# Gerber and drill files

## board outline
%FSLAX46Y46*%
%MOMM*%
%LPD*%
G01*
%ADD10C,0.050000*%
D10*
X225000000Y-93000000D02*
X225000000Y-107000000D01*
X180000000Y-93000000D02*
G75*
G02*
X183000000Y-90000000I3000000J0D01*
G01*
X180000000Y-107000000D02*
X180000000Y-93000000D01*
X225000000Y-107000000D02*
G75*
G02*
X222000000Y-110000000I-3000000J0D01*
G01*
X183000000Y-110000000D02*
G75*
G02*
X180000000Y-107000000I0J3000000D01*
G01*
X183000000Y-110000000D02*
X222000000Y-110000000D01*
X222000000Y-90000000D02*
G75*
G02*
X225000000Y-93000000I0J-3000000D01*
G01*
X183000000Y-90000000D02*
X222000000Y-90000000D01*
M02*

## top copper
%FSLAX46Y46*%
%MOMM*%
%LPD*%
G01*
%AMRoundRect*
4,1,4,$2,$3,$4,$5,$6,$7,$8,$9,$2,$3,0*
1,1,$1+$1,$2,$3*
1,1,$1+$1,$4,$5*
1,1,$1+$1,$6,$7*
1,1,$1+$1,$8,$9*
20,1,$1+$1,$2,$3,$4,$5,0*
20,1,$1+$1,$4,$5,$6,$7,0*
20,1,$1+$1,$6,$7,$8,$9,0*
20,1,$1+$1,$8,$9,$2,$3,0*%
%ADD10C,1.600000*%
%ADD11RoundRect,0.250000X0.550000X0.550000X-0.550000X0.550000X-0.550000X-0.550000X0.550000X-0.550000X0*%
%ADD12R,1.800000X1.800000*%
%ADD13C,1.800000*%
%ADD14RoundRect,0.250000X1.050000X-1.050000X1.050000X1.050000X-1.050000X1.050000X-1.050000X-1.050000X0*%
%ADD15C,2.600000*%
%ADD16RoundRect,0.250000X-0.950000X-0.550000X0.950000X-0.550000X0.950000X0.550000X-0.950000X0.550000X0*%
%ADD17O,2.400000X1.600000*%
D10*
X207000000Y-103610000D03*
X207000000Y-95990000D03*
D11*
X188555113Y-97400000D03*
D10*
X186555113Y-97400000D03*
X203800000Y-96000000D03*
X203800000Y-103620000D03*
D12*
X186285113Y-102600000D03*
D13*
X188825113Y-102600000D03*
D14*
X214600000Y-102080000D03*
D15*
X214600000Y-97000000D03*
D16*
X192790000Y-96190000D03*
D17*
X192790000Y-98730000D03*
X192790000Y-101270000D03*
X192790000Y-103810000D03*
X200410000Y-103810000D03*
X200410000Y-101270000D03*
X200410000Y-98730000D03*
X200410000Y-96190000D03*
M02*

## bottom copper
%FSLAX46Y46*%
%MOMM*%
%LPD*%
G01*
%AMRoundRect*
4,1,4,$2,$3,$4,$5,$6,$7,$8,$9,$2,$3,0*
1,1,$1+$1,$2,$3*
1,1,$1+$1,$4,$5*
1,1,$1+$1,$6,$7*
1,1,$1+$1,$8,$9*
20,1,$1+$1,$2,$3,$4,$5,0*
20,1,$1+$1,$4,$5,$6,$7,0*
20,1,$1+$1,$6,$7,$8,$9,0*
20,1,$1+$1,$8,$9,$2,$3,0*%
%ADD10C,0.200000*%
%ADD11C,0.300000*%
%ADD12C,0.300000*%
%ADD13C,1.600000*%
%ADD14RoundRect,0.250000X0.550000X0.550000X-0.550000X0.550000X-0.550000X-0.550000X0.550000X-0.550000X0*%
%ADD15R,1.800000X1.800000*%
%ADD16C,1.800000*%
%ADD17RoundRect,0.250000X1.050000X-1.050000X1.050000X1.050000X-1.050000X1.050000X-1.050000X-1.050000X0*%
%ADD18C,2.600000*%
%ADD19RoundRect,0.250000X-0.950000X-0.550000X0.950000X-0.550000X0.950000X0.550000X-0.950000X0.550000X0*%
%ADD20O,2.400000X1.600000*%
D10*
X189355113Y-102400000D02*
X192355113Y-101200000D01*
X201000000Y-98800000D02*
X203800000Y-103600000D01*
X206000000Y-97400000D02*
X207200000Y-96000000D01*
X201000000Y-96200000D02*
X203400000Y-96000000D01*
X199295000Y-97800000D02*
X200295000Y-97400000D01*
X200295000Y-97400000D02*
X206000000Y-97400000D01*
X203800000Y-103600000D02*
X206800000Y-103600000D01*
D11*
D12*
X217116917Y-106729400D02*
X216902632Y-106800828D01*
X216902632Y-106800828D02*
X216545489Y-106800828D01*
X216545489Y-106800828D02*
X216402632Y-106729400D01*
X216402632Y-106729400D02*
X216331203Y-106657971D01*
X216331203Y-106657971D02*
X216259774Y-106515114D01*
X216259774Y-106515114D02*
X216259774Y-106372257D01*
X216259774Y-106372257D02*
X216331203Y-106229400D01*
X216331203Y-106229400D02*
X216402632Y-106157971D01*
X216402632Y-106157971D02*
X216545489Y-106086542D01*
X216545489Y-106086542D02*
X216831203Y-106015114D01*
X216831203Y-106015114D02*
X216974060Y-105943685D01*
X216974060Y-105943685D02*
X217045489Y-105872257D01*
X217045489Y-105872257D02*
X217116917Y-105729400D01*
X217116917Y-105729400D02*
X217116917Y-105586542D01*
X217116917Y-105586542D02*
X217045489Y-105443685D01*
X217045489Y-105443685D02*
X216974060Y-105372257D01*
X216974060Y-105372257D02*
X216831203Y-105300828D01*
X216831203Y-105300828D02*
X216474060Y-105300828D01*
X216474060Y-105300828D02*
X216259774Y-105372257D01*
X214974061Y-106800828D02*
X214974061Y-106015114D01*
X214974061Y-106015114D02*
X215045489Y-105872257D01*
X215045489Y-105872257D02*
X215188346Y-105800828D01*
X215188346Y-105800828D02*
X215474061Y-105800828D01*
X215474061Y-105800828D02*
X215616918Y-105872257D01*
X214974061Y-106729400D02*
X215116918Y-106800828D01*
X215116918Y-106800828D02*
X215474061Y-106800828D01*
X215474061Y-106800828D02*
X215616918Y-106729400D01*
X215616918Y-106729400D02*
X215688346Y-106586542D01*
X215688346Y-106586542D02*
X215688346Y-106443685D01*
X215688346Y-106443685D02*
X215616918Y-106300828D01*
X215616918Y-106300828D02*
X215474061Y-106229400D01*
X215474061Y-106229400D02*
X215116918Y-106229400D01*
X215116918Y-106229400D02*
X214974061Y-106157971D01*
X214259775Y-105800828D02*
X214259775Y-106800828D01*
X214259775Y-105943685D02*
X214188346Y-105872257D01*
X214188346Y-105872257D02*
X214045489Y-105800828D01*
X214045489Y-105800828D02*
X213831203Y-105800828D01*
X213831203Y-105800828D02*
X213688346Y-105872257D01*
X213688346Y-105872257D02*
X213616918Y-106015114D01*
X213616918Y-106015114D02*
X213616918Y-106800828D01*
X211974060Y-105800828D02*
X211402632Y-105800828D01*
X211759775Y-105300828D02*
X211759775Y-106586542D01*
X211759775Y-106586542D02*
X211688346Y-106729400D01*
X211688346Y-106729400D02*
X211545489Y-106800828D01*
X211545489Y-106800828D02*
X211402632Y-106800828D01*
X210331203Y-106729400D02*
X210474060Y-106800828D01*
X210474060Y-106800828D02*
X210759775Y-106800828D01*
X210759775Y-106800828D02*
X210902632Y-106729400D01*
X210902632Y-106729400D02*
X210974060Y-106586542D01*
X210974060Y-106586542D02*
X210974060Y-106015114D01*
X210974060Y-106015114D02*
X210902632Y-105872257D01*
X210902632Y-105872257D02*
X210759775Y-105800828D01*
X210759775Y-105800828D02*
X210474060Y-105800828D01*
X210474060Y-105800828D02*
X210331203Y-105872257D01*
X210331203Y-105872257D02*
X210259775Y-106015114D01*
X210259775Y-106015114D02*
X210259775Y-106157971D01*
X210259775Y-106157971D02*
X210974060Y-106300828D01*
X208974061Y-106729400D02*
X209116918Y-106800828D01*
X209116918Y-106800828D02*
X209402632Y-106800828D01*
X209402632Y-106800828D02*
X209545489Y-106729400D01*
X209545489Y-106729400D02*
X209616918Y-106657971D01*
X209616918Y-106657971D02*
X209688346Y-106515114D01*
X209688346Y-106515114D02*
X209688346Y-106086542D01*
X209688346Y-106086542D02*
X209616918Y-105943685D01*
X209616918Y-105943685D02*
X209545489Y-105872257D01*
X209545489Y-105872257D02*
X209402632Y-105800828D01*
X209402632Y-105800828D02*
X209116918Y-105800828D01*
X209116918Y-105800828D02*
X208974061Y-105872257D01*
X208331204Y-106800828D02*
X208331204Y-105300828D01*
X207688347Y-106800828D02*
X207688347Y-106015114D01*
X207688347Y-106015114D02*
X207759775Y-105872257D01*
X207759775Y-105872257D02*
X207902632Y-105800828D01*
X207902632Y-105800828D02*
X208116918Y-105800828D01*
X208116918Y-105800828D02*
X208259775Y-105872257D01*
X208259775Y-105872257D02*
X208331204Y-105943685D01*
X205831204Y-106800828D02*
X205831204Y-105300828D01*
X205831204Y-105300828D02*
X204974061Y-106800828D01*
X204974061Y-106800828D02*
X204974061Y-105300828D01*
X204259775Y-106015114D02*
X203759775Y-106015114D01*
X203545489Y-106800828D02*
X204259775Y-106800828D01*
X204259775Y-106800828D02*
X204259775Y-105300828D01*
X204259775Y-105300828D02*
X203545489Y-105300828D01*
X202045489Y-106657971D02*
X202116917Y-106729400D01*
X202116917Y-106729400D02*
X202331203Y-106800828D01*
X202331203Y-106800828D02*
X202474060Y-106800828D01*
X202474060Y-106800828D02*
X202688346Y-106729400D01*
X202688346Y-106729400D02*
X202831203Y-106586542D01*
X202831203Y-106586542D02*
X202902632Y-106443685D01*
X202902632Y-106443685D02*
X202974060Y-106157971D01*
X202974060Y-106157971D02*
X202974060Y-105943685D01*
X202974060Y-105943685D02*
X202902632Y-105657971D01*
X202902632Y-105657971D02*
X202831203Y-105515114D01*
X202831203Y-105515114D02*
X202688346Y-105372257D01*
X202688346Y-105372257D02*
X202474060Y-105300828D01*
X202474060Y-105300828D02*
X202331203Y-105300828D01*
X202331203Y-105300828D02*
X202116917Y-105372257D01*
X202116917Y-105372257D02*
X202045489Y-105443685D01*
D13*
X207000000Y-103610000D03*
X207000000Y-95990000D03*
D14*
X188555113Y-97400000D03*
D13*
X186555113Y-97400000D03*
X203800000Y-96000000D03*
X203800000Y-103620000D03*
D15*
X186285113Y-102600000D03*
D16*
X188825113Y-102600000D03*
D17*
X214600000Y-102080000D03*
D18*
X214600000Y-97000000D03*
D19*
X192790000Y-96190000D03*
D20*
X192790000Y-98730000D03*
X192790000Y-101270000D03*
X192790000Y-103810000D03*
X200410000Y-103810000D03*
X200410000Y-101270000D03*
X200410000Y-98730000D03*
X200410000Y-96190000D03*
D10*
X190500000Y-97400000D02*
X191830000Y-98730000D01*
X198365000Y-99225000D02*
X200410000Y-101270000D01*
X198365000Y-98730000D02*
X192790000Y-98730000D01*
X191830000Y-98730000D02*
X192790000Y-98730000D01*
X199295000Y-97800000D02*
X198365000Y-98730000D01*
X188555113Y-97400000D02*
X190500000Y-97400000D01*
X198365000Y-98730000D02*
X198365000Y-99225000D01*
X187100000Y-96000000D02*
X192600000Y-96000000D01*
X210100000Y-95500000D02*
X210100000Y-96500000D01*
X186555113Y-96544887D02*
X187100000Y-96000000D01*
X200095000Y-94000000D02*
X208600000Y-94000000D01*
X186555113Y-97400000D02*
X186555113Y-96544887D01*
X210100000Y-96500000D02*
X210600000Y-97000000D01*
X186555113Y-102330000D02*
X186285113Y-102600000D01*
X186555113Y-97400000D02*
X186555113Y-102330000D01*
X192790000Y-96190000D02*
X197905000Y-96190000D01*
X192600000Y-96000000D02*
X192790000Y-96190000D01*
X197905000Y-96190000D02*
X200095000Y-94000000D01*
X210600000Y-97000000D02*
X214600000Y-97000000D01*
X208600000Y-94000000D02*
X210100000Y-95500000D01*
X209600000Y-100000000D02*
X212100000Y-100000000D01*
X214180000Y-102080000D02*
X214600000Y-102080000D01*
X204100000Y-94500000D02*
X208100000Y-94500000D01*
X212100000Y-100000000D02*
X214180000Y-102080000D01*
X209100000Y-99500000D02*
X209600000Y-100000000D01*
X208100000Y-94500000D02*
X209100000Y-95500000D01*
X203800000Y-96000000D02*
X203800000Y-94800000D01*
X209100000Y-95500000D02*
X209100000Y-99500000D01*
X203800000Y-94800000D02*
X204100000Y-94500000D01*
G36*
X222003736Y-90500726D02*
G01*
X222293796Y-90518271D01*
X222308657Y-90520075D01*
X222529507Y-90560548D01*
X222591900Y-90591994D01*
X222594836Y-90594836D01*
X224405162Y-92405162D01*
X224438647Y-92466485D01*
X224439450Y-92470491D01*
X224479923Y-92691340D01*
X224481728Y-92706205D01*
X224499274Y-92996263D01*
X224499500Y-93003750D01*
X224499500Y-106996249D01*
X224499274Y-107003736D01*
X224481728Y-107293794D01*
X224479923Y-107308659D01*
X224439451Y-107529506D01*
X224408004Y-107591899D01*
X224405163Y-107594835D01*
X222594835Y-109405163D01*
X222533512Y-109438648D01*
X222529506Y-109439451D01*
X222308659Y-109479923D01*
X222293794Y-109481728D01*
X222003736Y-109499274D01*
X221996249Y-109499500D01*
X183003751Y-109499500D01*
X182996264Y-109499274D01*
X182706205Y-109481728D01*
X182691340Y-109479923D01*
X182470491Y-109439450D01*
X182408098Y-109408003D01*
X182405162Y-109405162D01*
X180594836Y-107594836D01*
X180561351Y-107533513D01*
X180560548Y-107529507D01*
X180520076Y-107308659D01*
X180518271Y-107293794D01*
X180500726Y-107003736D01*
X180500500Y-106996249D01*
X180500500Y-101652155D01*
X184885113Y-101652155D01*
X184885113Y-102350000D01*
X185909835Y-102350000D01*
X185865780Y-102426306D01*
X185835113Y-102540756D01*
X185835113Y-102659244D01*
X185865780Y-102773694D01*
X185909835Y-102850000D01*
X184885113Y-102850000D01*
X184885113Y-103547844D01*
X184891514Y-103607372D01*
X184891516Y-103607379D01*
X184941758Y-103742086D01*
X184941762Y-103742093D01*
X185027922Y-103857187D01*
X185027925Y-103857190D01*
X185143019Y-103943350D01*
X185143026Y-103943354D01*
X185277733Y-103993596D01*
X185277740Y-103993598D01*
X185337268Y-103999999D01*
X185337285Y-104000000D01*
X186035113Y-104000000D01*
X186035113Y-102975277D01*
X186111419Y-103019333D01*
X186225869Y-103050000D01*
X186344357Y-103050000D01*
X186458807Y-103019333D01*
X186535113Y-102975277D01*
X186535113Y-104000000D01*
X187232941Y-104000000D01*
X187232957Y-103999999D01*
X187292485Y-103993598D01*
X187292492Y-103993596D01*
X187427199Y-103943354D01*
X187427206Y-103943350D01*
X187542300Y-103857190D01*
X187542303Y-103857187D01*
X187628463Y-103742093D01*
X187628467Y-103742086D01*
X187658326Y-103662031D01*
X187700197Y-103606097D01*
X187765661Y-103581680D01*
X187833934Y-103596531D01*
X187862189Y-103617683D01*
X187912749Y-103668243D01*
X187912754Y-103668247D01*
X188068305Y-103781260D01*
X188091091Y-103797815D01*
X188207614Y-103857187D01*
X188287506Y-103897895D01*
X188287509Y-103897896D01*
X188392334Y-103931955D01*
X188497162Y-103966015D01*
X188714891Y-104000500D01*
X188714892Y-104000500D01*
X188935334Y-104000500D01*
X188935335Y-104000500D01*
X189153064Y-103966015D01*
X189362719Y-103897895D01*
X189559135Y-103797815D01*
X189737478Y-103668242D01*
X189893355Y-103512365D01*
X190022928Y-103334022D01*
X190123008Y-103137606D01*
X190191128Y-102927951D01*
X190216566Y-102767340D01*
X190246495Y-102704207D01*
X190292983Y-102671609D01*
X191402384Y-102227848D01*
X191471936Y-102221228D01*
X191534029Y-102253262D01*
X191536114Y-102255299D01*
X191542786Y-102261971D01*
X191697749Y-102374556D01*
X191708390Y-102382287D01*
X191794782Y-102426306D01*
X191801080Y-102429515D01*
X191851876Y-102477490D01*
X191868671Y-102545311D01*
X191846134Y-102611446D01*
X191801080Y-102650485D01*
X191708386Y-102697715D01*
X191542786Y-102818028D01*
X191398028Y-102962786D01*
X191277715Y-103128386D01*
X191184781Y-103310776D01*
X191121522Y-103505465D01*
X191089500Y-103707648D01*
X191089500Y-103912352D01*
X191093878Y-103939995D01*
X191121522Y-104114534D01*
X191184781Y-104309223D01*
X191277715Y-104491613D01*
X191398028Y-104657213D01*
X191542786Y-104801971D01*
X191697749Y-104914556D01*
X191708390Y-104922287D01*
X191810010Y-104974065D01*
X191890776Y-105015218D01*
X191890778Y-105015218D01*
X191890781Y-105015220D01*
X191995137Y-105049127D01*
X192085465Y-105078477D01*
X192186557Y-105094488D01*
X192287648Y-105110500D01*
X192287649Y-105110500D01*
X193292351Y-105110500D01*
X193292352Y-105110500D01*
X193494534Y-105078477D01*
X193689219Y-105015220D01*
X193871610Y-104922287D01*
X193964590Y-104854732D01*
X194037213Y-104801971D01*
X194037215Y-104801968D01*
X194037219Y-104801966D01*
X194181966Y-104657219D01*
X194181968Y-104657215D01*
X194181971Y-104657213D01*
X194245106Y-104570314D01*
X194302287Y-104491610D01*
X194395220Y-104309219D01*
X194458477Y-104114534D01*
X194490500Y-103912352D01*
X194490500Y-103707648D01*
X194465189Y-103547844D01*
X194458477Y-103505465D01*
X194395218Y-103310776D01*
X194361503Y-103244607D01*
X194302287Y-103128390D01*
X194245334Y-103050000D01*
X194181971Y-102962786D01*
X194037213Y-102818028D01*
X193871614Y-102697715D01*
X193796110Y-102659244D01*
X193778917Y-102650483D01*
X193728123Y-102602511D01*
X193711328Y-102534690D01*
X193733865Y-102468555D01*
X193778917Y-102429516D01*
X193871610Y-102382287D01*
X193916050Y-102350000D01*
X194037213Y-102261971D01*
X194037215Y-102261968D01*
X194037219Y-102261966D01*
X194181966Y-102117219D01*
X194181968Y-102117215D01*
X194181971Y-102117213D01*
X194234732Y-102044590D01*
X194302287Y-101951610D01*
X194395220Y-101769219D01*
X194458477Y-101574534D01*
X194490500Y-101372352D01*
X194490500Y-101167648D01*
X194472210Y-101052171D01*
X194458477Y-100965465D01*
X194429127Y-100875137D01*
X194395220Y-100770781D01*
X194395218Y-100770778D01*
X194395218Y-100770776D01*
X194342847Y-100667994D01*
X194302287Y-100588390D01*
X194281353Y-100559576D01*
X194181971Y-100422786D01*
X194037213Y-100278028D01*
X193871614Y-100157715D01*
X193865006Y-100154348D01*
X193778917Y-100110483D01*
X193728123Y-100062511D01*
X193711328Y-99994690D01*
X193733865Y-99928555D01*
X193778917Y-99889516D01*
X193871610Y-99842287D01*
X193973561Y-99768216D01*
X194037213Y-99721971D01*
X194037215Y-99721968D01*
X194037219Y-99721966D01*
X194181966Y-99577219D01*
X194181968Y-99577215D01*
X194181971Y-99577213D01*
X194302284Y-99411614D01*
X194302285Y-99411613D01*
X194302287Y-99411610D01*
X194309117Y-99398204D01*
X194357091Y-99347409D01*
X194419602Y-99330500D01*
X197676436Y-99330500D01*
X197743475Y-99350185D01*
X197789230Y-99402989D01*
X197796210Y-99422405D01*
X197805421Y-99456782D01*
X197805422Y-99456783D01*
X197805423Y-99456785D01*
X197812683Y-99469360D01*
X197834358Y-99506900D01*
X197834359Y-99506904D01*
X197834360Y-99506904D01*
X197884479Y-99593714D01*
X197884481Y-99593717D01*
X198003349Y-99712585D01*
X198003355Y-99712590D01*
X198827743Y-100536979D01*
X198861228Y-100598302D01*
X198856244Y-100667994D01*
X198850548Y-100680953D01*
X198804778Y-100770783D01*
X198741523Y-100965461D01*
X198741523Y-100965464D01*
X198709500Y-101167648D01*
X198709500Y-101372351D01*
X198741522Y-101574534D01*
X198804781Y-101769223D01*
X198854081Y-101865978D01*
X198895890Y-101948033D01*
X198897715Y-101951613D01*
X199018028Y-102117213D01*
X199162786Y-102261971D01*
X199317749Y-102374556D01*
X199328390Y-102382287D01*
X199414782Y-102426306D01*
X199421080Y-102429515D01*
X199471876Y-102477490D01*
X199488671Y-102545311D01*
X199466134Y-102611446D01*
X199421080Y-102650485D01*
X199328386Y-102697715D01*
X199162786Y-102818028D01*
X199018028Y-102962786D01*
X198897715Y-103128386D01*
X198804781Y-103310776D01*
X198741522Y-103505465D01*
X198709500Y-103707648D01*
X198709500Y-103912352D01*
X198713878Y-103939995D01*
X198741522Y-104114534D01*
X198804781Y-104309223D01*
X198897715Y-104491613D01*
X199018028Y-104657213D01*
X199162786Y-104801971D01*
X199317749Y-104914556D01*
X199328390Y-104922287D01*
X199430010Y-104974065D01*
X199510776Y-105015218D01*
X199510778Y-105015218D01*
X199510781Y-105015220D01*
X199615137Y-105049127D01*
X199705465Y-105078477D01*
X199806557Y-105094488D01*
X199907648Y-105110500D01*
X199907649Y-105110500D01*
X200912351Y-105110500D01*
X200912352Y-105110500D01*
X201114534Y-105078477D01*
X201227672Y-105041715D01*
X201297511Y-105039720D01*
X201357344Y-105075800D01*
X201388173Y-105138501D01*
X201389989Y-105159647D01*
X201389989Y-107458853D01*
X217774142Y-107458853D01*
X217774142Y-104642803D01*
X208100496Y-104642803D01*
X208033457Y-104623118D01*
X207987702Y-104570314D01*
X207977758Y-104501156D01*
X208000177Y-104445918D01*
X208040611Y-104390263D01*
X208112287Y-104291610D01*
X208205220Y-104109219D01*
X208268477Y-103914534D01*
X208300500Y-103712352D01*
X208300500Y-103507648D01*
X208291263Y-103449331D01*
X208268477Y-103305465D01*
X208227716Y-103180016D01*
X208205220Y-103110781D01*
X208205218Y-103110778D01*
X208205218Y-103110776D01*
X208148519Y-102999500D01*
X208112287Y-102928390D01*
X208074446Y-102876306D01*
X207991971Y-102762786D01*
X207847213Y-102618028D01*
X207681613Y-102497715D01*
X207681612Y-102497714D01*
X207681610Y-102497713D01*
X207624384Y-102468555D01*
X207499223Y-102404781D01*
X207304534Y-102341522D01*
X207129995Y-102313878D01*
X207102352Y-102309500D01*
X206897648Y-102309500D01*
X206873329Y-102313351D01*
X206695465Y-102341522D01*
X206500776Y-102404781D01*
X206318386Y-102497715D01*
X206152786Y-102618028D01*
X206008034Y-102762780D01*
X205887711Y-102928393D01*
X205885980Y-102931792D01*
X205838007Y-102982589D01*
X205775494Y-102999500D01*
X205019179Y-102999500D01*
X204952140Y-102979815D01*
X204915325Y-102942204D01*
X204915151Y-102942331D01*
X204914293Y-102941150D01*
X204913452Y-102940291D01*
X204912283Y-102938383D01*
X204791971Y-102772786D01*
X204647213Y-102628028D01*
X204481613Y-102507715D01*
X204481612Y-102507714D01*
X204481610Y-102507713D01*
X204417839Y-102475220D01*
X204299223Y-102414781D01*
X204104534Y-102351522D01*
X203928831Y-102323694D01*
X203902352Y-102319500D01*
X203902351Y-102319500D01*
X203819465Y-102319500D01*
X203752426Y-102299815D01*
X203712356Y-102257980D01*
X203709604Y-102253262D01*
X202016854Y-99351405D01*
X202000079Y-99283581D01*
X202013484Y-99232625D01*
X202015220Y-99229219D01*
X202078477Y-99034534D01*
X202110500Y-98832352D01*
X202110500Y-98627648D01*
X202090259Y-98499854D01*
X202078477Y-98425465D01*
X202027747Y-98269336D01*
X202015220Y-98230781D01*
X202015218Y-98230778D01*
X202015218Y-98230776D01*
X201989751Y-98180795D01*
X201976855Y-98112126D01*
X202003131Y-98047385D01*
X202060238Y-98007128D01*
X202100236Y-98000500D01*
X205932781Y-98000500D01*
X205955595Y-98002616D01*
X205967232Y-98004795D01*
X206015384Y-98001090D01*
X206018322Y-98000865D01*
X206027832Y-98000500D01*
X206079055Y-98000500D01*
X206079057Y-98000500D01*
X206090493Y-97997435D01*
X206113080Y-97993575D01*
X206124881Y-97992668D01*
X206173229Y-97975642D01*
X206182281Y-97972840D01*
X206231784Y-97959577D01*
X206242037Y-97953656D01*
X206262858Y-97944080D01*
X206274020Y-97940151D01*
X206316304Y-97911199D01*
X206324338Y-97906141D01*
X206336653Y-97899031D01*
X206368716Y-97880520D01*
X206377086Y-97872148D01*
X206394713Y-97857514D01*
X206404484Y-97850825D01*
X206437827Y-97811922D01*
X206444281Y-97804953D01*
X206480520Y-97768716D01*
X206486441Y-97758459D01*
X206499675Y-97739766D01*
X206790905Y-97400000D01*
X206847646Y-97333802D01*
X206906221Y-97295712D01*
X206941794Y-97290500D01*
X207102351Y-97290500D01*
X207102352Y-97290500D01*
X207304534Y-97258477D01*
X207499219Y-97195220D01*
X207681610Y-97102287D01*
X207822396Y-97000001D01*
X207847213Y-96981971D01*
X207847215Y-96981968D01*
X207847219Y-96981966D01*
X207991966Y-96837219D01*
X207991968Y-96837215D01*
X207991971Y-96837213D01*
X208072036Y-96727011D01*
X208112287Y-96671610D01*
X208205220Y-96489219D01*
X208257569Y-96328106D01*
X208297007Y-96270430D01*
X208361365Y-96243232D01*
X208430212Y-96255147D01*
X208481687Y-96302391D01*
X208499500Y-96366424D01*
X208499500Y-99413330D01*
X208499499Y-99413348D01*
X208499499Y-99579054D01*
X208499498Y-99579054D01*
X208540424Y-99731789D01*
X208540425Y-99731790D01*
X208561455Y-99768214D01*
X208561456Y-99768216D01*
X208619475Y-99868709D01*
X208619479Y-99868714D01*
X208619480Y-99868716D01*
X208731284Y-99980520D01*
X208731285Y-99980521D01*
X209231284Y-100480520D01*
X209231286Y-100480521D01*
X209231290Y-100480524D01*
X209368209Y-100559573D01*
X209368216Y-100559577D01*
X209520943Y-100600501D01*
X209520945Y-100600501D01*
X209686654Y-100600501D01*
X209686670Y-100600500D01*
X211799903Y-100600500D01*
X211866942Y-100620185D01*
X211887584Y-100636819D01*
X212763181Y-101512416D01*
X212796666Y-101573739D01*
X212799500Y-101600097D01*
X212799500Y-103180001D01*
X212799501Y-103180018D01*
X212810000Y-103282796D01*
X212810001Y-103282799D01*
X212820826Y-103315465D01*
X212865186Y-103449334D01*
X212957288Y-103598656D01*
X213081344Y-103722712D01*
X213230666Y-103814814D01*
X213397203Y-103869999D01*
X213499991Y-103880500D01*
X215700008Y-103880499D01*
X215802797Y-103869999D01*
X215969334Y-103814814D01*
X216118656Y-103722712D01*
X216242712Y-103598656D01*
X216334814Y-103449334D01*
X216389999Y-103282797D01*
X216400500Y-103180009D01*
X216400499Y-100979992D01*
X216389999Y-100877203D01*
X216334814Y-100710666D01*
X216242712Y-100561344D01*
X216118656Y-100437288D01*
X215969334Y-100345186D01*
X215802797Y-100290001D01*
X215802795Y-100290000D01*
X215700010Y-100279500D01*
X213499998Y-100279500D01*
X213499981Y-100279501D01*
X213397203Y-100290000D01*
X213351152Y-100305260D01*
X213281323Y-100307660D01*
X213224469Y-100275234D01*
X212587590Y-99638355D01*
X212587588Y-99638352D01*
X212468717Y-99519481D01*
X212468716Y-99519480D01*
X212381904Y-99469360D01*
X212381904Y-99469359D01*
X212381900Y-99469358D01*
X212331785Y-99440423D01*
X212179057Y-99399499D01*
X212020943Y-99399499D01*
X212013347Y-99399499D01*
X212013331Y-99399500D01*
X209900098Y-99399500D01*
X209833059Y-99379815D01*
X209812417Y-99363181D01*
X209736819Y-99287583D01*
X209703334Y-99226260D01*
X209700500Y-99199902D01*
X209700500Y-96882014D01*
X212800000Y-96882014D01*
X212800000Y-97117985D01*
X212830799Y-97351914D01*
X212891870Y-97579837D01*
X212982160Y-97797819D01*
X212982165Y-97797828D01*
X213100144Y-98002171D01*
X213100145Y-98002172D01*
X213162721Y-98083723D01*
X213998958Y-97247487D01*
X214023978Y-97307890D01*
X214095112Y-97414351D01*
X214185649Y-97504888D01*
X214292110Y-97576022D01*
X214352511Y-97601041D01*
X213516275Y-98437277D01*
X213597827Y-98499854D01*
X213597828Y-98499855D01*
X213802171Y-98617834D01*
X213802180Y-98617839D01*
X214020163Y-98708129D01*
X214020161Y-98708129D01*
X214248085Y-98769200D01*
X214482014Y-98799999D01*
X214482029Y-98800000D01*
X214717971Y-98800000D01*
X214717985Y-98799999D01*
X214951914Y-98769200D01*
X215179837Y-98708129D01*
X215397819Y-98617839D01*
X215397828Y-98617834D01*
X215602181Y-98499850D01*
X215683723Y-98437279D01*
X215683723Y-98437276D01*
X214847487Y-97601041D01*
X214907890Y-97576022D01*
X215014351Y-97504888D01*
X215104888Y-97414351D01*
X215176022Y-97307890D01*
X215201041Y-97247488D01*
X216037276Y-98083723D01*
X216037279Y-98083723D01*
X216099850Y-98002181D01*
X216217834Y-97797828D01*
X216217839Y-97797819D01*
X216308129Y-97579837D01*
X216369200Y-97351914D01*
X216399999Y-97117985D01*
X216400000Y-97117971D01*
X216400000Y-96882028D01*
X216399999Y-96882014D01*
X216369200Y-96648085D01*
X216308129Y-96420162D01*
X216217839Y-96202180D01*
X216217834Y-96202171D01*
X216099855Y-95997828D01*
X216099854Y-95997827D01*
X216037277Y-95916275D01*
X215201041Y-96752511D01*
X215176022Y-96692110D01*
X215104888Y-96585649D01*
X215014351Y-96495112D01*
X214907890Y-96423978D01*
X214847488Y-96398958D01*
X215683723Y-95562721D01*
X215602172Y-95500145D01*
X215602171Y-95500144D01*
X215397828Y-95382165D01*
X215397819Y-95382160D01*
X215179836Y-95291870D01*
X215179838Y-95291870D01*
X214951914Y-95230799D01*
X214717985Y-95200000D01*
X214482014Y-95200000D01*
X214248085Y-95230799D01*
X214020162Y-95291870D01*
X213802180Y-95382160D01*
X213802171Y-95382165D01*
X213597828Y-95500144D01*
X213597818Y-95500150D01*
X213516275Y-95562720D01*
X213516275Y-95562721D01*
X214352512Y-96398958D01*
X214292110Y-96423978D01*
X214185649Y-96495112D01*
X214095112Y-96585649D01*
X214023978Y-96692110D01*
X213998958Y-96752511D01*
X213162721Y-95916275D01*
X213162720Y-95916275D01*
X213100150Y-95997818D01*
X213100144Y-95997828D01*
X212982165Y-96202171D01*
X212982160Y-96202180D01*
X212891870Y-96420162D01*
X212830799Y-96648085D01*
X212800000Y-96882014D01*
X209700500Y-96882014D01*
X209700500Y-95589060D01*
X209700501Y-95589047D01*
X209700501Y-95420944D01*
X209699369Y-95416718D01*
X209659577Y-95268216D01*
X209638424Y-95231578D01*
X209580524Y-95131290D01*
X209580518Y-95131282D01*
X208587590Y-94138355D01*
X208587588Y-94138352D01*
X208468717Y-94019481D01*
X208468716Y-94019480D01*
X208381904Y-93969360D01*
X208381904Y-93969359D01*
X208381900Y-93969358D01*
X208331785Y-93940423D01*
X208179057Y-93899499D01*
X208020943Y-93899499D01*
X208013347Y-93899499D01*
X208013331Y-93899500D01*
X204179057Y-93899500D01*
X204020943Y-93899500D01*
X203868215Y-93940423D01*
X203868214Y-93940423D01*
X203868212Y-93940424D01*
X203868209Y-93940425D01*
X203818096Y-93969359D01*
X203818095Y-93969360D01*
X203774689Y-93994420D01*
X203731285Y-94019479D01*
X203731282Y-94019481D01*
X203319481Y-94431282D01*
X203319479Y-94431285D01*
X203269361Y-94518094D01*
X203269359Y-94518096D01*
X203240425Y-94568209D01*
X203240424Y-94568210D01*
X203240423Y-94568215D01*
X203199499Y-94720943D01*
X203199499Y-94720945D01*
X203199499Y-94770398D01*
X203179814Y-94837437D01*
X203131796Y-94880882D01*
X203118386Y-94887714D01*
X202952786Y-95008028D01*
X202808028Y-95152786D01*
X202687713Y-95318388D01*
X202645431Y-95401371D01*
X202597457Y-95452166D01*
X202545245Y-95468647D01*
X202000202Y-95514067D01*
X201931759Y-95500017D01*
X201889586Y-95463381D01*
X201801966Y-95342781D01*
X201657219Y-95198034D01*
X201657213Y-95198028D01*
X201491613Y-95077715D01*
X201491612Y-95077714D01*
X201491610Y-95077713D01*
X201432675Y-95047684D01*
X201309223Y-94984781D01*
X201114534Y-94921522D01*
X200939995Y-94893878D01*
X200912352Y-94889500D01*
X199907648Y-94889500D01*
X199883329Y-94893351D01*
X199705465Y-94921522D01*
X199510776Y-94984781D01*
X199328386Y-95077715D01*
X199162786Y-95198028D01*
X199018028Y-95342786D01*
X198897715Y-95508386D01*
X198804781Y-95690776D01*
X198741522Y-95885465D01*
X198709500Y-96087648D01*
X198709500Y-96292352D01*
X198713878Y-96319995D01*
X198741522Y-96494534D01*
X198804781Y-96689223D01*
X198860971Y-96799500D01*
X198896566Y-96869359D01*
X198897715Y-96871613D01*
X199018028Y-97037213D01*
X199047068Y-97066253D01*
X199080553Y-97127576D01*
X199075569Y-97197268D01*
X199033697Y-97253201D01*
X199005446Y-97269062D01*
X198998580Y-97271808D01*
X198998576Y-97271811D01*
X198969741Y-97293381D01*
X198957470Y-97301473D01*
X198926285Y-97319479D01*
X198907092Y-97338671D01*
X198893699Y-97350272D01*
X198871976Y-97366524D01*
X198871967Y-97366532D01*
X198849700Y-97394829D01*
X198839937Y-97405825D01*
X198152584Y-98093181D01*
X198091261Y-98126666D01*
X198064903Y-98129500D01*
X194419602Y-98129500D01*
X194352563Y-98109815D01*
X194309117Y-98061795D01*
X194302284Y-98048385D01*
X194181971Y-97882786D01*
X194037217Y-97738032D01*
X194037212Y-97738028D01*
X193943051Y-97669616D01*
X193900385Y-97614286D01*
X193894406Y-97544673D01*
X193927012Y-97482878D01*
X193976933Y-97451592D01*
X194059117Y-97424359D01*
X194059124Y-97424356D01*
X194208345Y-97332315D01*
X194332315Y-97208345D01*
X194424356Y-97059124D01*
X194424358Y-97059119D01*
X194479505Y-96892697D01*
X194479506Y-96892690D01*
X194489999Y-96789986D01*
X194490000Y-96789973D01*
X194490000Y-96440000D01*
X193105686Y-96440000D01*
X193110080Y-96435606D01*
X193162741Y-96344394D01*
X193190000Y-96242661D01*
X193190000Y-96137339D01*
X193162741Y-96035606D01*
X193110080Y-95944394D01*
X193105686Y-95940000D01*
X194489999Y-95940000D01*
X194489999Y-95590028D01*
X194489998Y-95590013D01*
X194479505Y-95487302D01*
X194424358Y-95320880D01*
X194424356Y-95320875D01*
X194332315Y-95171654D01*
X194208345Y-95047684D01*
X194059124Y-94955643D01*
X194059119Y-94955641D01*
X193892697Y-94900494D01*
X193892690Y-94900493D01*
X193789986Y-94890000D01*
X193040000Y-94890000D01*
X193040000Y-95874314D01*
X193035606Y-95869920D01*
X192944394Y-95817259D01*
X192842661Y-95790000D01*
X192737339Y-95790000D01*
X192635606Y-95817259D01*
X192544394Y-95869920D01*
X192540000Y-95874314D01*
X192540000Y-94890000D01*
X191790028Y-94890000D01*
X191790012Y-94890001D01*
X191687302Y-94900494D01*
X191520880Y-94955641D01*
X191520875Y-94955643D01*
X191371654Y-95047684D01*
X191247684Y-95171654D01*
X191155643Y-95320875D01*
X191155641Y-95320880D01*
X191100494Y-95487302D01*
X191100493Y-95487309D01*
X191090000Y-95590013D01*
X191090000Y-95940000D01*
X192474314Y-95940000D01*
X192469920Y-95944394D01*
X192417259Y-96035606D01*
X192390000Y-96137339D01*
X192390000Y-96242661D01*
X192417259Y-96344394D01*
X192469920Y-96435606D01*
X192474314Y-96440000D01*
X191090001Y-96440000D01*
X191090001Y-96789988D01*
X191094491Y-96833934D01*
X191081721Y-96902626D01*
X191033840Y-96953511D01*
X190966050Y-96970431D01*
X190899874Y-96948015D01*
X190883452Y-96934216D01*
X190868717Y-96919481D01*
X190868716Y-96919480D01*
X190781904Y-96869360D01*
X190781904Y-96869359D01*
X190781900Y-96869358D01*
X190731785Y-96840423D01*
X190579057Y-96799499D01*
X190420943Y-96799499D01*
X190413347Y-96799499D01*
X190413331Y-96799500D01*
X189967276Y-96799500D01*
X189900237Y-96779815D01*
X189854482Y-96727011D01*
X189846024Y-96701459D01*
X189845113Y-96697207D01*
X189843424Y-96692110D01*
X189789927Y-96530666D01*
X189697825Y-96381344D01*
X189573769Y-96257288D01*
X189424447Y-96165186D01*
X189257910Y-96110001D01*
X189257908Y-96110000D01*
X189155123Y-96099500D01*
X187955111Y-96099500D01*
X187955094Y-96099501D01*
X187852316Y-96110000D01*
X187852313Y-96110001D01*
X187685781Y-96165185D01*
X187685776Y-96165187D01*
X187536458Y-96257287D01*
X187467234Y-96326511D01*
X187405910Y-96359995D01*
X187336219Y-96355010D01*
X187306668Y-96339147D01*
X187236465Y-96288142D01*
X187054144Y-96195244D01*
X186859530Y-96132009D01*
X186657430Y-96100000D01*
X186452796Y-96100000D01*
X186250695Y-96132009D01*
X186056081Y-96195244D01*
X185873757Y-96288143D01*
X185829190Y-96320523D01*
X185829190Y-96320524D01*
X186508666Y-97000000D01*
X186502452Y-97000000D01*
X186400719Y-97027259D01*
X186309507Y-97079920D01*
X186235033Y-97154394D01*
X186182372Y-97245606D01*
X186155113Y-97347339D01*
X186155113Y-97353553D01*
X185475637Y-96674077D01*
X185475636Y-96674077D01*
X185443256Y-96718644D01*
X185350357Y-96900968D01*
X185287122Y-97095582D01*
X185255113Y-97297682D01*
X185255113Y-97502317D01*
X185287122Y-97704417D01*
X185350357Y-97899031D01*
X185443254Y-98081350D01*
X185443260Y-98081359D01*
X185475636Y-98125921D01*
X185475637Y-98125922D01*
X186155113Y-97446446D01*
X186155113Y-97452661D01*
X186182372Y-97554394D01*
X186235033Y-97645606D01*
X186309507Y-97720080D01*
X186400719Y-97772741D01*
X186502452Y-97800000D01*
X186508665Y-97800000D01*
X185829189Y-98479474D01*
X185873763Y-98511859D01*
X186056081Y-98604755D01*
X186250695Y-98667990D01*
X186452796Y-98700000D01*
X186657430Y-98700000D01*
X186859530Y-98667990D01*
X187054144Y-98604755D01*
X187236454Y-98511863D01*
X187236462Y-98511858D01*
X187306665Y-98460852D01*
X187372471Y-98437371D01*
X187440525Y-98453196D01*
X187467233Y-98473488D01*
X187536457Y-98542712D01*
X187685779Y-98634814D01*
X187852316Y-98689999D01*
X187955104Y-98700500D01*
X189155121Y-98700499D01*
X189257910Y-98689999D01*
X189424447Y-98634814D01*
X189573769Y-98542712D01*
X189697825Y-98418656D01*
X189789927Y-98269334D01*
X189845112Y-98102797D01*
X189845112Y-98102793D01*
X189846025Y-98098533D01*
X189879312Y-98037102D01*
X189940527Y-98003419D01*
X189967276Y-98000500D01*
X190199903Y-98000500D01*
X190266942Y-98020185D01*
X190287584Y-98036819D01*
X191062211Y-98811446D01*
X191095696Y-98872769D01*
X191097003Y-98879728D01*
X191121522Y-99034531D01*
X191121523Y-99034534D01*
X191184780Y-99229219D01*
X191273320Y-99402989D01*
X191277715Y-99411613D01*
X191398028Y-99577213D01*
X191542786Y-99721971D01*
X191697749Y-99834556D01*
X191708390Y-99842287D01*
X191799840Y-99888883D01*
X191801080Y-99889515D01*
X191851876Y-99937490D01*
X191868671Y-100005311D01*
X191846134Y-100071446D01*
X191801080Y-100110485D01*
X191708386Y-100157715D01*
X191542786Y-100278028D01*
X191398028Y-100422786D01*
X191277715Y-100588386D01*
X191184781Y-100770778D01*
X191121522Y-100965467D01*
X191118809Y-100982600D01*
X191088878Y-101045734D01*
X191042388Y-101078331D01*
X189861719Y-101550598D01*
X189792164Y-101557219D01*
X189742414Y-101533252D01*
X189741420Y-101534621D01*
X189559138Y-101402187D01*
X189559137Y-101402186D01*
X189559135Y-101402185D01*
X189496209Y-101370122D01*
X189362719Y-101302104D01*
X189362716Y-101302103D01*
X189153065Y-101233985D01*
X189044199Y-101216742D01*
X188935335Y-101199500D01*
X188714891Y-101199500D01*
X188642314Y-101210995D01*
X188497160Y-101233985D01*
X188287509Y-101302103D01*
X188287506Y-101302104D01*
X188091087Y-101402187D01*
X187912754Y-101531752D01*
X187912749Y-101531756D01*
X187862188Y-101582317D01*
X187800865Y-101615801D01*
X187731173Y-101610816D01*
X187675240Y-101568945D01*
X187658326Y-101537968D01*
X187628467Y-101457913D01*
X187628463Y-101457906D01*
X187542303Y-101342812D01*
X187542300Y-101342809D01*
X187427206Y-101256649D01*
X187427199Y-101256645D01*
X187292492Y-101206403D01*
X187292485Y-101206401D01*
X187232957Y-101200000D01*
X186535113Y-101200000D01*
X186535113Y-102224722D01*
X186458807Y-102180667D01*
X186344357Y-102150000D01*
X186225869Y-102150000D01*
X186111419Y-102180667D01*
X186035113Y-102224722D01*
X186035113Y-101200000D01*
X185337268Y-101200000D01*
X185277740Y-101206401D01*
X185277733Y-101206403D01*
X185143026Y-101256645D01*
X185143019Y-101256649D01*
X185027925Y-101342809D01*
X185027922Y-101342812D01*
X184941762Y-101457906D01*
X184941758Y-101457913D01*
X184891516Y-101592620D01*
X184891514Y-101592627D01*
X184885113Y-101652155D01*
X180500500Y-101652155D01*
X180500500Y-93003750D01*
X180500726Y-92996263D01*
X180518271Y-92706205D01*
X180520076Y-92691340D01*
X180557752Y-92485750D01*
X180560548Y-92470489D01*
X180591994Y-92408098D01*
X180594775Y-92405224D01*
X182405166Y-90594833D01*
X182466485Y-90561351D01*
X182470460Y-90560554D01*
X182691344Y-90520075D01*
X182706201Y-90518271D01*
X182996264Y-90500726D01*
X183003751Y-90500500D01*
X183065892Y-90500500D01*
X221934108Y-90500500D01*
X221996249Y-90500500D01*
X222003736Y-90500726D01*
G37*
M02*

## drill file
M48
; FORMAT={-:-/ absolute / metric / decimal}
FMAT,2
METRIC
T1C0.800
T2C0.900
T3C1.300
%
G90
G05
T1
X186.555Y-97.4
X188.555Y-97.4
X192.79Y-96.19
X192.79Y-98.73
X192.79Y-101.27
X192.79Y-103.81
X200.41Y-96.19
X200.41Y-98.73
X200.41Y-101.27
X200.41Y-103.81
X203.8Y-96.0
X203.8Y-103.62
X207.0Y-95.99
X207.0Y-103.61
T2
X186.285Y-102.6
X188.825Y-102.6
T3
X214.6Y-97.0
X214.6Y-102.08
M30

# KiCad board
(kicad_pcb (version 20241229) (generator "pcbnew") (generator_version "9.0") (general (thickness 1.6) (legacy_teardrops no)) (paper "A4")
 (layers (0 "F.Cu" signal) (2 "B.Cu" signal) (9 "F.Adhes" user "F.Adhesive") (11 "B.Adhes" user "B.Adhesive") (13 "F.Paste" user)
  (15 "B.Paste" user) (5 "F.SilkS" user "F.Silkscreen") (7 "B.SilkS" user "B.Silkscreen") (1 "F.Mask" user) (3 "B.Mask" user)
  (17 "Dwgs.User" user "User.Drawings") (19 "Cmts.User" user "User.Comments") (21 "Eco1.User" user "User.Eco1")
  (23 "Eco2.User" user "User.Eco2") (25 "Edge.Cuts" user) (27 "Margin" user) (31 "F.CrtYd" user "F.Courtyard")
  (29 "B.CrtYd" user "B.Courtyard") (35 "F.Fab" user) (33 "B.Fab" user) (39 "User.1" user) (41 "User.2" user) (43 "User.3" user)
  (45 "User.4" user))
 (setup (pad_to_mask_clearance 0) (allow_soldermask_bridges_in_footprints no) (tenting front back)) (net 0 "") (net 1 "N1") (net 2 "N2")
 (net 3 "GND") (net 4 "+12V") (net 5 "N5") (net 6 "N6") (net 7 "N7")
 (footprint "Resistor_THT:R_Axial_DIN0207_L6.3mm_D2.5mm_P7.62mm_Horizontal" (layer "F.Cu") (at 207 103.61 90)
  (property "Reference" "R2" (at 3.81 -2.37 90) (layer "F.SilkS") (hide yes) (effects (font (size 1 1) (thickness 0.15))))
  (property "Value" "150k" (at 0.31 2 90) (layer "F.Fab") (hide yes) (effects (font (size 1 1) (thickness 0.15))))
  (pad "1" thru_hole circle (at 0 0 90) (size 1.6 1.6) (drill 0.8) (layers "*.Cu" "*.Mask") (remove_unused_layers no) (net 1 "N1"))
  (pad "2" thru_hole circle (at 7.62 0 90) (size 1.6 1.6) (drill 0.8) (layers "*.Cu" "*.Mask") (remove_unused_layers no) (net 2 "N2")))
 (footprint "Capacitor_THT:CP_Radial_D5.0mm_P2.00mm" (layer "F.Cu") (at 188.555113 97.4 180)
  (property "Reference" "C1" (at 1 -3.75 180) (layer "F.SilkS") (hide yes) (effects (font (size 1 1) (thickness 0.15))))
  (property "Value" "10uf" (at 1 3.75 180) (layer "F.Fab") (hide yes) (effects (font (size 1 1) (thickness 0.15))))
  (pad "1" thru_hole roundrect (at 0 0 180) (size 1.6 1.6) (drill 0.8) (layers "*.Cu" "*.Mask") (remove_unused_layers no)
   (roundrect_rratio 0.15625) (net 2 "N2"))
  (pad "2" thru_hole circle (at 2 0 180) (size 1.6 1.6) (drill 0.8) (layers "*.Cu" "*.Mask") (remove_unused_layers no) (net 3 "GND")))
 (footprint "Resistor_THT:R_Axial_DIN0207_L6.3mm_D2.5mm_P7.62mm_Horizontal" (layer "F.Cu") (at 203.8 96 -90)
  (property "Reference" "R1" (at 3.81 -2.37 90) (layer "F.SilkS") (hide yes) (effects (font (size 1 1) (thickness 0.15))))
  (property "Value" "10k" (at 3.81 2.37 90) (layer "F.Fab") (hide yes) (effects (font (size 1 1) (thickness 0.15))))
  (pad "1" thru_hole circle (at 0 0 270) (size 1.6 1.6) (drill 0.8) (layers "*.Cu" "*.Mask") (remove_unused_layers no) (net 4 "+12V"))
  (pad "2" thru_hole circle (at 7.62 0 270) (size 1.6 1.6) (drill 0.8) (layers "*.Cu" "*.Mask") (remove_unused_layers no) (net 1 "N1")))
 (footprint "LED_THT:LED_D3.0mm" (layer "F.Cu") (at 186.285113 102.6)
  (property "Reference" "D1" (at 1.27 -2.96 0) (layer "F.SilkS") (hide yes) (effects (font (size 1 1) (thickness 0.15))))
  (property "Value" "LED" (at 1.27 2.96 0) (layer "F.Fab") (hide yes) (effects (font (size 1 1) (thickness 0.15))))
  (pad "1" thru_hole rect (at 0 0) (size 1.8 1.8) (drill 0.9) (layers "*.Cu" "*.Mask") (remove_unused_layers no) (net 3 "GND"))
  (pad "2" thru_hole circle (at 2.54 0) (size 1.8 1.8) (drill 0.9) (layers "*.Cu" "*.Mask") (remove_unused_layers no) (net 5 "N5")))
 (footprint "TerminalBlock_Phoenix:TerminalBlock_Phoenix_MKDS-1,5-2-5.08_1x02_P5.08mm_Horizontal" (layer "F.Cu") (at 214.6 102.08 90)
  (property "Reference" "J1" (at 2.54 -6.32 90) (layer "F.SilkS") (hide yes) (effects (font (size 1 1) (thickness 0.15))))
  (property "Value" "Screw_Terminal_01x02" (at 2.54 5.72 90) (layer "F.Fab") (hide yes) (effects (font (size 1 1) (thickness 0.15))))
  (pad "1" thru_hole roundrect (at 0 0 90) (size 2.6 2.6) (drill 1.3) (layers "*.Cu" "*.Mask") (remove_unused_layers no)
   (roundrect_rratio 0.096154) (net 4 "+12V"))
  (pad "2" thru_hole circle (at 5.08 0 90) (size 2.6 2.6) (drill 1.3) (layers "*.Cu" "*.Mask") (remove_unused_layers no) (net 3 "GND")))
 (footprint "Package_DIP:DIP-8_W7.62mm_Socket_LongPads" (layer "F.Cu") (at 192.79 96.19)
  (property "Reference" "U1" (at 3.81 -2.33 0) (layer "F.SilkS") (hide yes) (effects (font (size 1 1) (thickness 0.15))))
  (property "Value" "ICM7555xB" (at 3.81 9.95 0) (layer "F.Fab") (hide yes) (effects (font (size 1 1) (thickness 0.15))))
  (pad "1" thru_hole roundrect (at 0 0) (size 2.4 1.6) (drill 0.8) (layers "*.Cu" "*.Mask") (remove_unused_layers no)
   (roundrect_rratio 0.15625) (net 3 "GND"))
  (pad "2" thru_hole oval (at 0 2.54) (size 2.4 1.6) (drill 0.8) (layers "*.Cu" "*.Mask") (remove_unused_layers no) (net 2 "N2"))
  (pad "3" thru_hole oval (at 0 5.08) (size 2.4 1.6) (drill 0.8) (layers "*.Cu" "*.Mask") (remove_unused_layers no) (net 5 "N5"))
  (pad "4" thru_hole oval (at 0 7.62) (size 2.4 1.6) (drill 0.8) (layers "*.Cu" "*.Mask") (remove_unused_layers no) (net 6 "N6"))
  (pad "5" thru_hole oval (at 7.62 7.62) (size 2.4 1.6) (drill 0.8) (layers "*.Cu" "*.Mask") (remove_unused_layers no) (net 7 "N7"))
  (pad "6" thru_hole oval (at 7.62 5.08) (size 2.4 1.6) (drill 0.8) (layers "*.Cu" "*.Mask") (remove_unused_layers no) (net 2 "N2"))
  (pad "7" thru_hole oval (at 7.62 2.54) (size 2.4 1.6) (drill 0.8) (layers "*.Cu" "*.Mask") (remove_unused_layers no) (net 1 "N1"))
  (pad "8" thru_hole oval (at 7.62 0) (size 2.4 1.6) (drill 0.8) (layers "*.Cu" "*.Mask") (remove_unused_layers no) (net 4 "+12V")))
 (gr_line (start 189.355113 102.4) (end 192.355113 101.2) (stroke (width 0.2) (type default)) (layer "B.Cu") (net 5))
 (gr_line (start 201 98.8) (end 203.8 103.6) (stroke (width 0.2) (type default)) (layer "B.Cu") (net 1))
 (gr_line (start 206 97.4) (end 207.2 96) (stroke (width 0.2) (type default)) (layer "B.Cu") (net 2))
 (gr_line (start 201 96.2) (end 203.4 96) (stroke (width 0.2) (type default)) (layer "B.Cu") (net 4))
 (gr_line (start 199.295 97.8) (end 200.295 97.4) (stroke (width 0.2) (type default)) (layer "B.Cu") (net 2))
 (gr_line (start 200.295 97.4) (end 206 97.4) (stroke (width 0.2) (type default)) (layer "B.Cu") (net 2))
 (gr_line (start 203.8 103.6) (end 206.8 103.6) (stroke (width 0.2) (type default)) (layer "B.Cu") (net 1))
 (gr_line (start 225 93) (end 225 107) (stroke (width 0.05) (type default)) (layer "Edge.Cuts"))
 (gr_arc (start 180 93) (mid 180.87868 90.87868) (end 183 90) (stroke (width 0.05) (type default)) (layer "Edge.Cuts"))
 (gr_line (start 180 107) (end 180 93) (stroke (width 0.05) (type default)) (layer "Edge.Cuts"))
 (gr_arc (start 225 107) (mid 224.12132 109.12132) (end 222 110) (stroke (width 0.05) (type default)) (layer "Edge.Cuts"))
 (gr_arc (start 183 110) (mid 180.87868 109.12132) (end 180 107) (stroke (width 0.05) (type default)) (layer "Edge.Cuts"))
 (gr_line (start 183 110) (end 222 110) (stroke (width 0.05) (type default)) (layer "Edge.Cuts"))
 (gr_arc (start 222 90) (mid 224.12132 90.87868) (end 225 93) (stroke (width 0.05) (type default)) (layer "Edge.Cuts"))
 (gr_line (start 183 90) (end 222 90) (stroke (width 0.05) (type default)) (layer "Edge.Cuts"))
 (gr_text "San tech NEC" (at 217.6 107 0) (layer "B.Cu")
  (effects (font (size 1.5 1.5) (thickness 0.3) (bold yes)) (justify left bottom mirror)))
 (segment (start 190.5 97.4) (end 191.83 98.73) (width 0.2) (layer "B.Cu") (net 2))
 (segment (start 198.365 99.225) (end 200.41 101.27) (width 0.2) (layer "B.Cu") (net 2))
 (segment (start 198.365 98.73) (end 192.79 98.73) (width 0.2) (layer "B.Cu") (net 2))
 (segment (start 191.83 98.73) (end 192.79 98.73) (width 0.2) (layer "B.Cu") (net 2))
 (segment (start 199.295 97.8) (end 198.365 98.73) (width 0.2) (layer "B.Cu") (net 2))
 (segment (start 188.555113 97.4) (end 190.5 97.4) (width 0.2) (layer "B.Cu") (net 2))
 (segment (start 198.365 98.73) (end 198.365 99.225) (width 0.2) (layer "B.Cu") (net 2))
 (segment (start 187.1 96) (end 192.6 96) (width 0.2) (layer "B.Cu") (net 3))
 (segment (start 210.1 95.5) (end 210.1 96.5) (width 0.2) (layer "B.Cu") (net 3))
 (segment (start 186.555113 96.544887) (end 187.1 96) (width 0.2) (layer "B.Cu") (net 3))
 (segment (start 200.095 94) (end 208.6 94) (width 0.2) (layer "B.Cu") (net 3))
 (segment (start 186.555113 97.4) (end 186.555113 96.544887) (width 0.2) (layer "B.Cu") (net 3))
 (segment (start 210.1 96.5) (end 210.6 97) (width 0.2) (layer "B.Cu") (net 3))
 (segment (start 186.555113 102.33) (end 186.285113 102.6) (width 0.2) (layer "B.Cu") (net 3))
 (segment (start 186.555113 97.4) (end 186.555113 102.33) (width 0.2) (layer "B.Cu") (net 3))
 (segment (start 192.79 96.19) (end 197.905 96.19) (width 0.2) (layer "B.Cu") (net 3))
 (segment (start 192.6 96) (end 192.79 96.19) (width 0.2) (layer "B.Cu") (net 3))
 (segment (start 197.905 96.19) (end 200.095 94) (width 0.2) (layer "B.Cu") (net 3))
 (segment (start 210.6 97) (end 214.6 97) (width 0.2) (layer "B.Cu") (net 3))
 (segment (start 208.6 94) (end 210.1 95.5) (width 0.2) (layer "B.Cu") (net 3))
 (segment (start 209.6 100) (end 212.1 100) (width 0.2) (layer "B.Cu") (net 4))
 (segment (start 214.18 102.08) (end 214.6 102.08) (width 0.2) (layer "B.Cu") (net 4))
 (segment (start 204.1 94.5) (end 208.1 94.5) (width 0.2) (layer "B.Cu") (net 4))
 (segment (start 212.1 100) (end 214.18 102.08) (width 0.2) (layer "B.Cu") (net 4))
 (segment (start 209.1 99.5) (end 209.6 100) (width 0.2) (layer "B.Cu") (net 4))
 (segment (start 208.1 94.5) (end 209.1 95.5) (width 0.2) (layer "B.Cu") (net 4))
 (segment (start 203.8 96) (end 203.8 94.8) (width 0.2) (layer "B.Cu") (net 4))
 (segment (start 209.1 95.5) (end 209.1 99.5) (width 0.2) (layer "B.Cu") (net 4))
 (segment (start 203.8 94.8) (end 204.1 94.5) (width 0.2) (layer "B.Cu") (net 4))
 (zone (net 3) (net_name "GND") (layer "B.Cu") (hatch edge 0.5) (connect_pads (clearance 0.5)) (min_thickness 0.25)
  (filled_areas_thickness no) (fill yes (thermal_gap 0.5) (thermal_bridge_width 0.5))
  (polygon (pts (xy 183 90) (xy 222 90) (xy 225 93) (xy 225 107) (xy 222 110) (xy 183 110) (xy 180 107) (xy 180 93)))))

